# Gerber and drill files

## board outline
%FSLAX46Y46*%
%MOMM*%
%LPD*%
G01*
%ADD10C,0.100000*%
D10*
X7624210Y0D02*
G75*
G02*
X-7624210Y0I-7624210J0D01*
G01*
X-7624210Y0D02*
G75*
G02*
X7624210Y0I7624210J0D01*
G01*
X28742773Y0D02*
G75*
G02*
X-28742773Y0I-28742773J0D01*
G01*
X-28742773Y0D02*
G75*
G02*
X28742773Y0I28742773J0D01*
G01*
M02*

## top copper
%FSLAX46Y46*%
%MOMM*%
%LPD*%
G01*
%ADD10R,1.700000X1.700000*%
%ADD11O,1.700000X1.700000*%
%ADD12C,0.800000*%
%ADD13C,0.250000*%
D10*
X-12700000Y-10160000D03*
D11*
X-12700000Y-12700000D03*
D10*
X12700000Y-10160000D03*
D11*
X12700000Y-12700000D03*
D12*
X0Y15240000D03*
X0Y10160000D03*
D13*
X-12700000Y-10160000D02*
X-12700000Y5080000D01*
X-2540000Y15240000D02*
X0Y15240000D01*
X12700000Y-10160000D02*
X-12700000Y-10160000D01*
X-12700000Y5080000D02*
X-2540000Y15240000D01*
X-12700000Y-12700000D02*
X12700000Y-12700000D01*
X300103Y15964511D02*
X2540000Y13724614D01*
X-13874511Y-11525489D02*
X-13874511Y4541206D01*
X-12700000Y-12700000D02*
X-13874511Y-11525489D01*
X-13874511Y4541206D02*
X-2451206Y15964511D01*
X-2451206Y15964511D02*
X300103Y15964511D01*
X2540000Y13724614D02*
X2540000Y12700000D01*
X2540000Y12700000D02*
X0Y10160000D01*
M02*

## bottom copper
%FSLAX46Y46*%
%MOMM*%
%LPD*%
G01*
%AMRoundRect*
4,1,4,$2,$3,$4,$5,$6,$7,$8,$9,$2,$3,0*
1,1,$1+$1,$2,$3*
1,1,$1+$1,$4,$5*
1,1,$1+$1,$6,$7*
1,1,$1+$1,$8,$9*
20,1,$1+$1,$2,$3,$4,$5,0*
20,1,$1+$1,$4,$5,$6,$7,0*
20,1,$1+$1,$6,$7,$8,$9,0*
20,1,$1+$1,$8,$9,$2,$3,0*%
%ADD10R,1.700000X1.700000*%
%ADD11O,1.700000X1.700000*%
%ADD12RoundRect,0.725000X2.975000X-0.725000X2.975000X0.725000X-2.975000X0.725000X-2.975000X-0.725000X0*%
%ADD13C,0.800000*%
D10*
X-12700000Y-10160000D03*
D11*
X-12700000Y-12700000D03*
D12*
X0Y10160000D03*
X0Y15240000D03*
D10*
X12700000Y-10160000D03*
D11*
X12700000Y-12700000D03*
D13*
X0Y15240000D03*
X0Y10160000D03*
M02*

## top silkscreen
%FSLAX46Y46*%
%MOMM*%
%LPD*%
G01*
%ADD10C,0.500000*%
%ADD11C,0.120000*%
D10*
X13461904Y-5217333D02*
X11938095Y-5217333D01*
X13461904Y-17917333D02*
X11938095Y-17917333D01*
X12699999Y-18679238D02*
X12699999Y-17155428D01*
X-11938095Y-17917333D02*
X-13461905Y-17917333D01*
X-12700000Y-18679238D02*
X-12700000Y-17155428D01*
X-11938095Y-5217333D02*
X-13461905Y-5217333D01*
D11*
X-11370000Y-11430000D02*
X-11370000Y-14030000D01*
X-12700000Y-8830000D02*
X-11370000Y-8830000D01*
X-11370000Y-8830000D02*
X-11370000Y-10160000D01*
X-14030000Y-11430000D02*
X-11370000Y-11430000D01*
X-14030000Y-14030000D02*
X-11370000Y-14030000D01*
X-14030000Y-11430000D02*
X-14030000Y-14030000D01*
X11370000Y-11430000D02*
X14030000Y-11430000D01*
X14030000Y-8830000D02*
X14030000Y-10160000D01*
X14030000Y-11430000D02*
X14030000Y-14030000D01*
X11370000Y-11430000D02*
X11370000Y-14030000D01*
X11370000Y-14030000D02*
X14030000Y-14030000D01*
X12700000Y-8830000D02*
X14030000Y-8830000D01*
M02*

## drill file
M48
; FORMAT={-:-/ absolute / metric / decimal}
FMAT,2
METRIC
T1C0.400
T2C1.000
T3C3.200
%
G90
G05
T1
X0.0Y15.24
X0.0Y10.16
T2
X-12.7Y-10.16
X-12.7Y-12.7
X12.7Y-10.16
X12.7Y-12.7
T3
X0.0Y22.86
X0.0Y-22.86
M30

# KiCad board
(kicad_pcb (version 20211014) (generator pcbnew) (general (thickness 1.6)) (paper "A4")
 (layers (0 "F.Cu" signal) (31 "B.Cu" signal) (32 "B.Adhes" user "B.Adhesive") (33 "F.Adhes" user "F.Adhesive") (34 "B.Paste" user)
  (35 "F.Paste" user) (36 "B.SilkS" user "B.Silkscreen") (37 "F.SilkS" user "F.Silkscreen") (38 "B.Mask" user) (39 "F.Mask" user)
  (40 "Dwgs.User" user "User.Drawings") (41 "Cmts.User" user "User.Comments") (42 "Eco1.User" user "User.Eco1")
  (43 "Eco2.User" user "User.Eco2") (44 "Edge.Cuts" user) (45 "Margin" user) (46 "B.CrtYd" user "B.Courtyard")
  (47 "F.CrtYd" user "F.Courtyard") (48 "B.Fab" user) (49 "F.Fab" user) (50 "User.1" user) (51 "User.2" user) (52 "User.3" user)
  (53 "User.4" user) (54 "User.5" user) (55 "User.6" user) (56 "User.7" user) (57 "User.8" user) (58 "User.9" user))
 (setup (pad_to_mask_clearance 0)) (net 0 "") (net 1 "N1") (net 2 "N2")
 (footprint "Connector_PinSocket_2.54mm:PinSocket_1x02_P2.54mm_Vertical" (layer "F.Cu") (at -12.7 10.16)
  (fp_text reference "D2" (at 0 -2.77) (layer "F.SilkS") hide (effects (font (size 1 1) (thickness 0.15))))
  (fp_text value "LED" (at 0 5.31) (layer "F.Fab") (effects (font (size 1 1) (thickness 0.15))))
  (fp_line (start 1.33 1.27) (end 1.33 3.87) (layer "F.SilkS") (width 0.12))
  (fp_line (start 0 -1.33) (end 1.33 -1.33) (layer "F.SilkS") (width 0.12))
  (fp_line (start 1.33 -1.33) (end 1.33 0) (layer "F.SilkS") (width 0.12))
  (fp_line (start -1.33 1.27) (end 1.33 1.27) (layer "F.SilkS") (width 0.12))
  (fp_line (start -1.33 3.87) (end 1.33 3.87) (layer "F.SilkS") (width 0.12))
  (fp_line (start -1.33 1.27) (end -1.33 3.87) (layer "F.SilkS") (width 0.12))
  (pad "1" thru_hole rect (at 0 0) (size 1.7 1.7) (drill 1) (layers *.Cu *.Mask) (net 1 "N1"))
  (pad "2" thru_hole oval (at 0 2.54) (size 1.7 1.7) (drill 1) (layers *.Cu *.Mask) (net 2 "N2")))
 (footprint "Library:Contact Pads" (layer "F.Cu") (at 0 0)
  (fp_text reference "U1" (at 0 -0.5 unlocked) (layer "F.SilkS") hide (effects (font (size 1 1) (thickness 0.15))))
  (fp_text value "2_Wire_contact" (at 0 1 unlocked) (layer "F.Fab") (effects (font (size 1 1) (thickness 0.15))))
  (pad "1" smd roundrect (at 0 -10.16 90) (size 2.9 7.4) (layers "B.Cu" "B.Paste" "B.Mask") (roundrect_rratio 0.25) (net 2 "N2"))
  (pad "2" smd roundrect (at 0 -15.24 90) (size 2.9 7.4) (layers "B.Cu" "B.Paste" "B.Mask") (roundrect_rratio 0.25) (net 1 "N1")))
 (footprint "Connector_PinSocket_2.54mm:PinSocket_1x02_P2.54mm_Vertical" (layer "F.Cu") (at 12.7 10.16)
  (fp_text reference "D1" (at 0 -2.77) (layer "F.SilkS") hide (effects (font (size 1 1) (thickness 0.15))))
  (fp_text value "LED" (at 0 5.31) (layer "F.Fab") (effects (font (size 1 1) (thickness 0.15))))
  (fp_line (start -1.33 1.27) (end 1.33 1.27) (layer "F.SilkS") (width 0.12))
  (fp_line (start 1.33 -1.33) (end 1.33 0) (layer "F.SilkS") (width 0.12))
  (fp_line (start 1.33 1.27) (end 1.33 3.87) (layer "F.SilkS") (width 0.12))
  (fp_line (start -1.33 1.27) (end -1.33 3.87) (layer "F.SilkS") (width 0.12))
  (fp_line (start -1.33 3.87) (end 1.33 3.87) (layer "F.SilkS") (width 0.12))
  (fp_line (start 0 -1.33) (end 1.33 -1.33) (layer "F.SilkS") (width 0.12))
  (pad "1" thru_hole rect (at 0 0) (size 1.7 1.7) (drill 1) (layers *.Cu *.Mask) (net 1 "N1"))
  (pad "2" thru_hole oval (at 0 2.54) (size 1.7 1.7) (drill 1) (layers *.Cu *.Mask) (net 2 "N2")))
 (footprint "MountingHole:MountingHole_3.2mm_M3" (layer "F.Cu") (at 0 -22.86)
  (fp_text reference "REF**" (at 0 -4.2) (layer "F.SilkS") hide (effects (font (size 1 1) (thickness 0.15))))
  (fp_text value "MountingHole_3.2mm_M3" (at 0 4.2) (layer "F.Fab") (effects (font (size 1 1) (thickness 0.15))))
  (pad "" np_thru_hole circle (at 0 0) (size 3.2 3.2) (drill 3.2) (layers *.Cu *.Mask)))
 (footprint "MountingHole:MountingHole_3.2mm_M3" (layer "F.Cu") (at 0 22.86)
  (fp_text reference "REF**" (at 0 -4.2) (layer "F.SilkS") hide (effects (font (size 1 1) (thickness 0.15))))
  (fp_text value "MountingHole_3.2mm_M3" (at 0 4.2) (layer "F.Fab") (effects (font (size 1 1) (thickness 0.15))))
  (pad "" np_thru_hole circle (at 0 0) (size 3.2 3.2) (drill 3.2) (layers *.Cu *.Mask)))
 (gr_circle (center 0 0) (end 7.62421 0) (layer "Edge.Cuts") (width 0.1) (fill none))
 (gr_circle (center 0 0) (end 28.742773 0) (layer "Edge.Cuts") (width 0.1) (fill none))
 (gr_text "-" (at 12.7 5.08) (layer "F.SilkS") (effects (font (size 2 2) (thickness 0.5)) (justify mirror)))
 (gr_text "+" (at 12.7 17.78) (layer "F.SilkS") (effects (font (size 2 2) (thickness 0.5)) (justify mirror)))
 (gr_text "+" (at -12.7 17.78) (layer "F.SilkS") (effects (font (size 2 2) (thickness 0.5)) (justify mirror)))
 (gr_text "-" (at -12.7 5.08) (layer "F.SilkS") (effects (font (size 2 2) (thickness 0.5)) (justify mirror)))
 (segment (start -12.7 10.16) (end -12.7 -5.08) (width 0.25) (layer "F.Cu") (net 1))
 (segment (start -2.54 -15.24) (end 0 -15.24) (width 0.25) (layer "F.Cu") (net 1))
 (segment (start 12.7 10.16) (end -12.7 10.16) (width 0.25) (layer "F.Cu") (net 1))
 (segment (start -12.7 -5.08) (end -2.54 -15.24) (width 0.25) (layer "F.Cu") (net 1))
 (via (at 0 -15.24) (size 0.8) (drill 0.4) (layers "F.Cu" "B.Cu") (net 1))
 (segment (start -12.7 12.7) (end 12.7 12.7) (width 0.25) (layer "F.Cu") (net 2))
 (segment (start 0.300103 -15.964511) (end 2.54 -13.724614) (width 0.25) (layer "F.Cu") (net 2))
 (segment (start -13.874511 11.525489) (end -13.874511 -4.541206) (width 0.25) (layer "F.Cu") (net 2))
 (segment (start -12.7 12.7) (end -13.874511 11.525489) (width 0.25) (layer "F.Cu") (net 2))
 (segment (start -13.874511 -4.541206) (end -2.451206 -15.964511) (width 0.25) (layer "F.Cu") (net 2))
 (segment (start -2.451206 -15.964511) (end 0.300103 -15.964511) (width 0.25) (layer "F.Cu") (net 2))
 (segment (start 2.54 -13.724614) (end 2.54 -12.7) (width 0.25) (layer "F.Cu") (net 2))
 (segment (start 2.54 -12.7) (end 0 -10.16) (width 0.25) (layer "F.Cu") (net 2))
 (via (at 0 -10.16) (size 0.8) (drill 0.4) (layers "F.Cu" "B.Cu") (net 2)))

